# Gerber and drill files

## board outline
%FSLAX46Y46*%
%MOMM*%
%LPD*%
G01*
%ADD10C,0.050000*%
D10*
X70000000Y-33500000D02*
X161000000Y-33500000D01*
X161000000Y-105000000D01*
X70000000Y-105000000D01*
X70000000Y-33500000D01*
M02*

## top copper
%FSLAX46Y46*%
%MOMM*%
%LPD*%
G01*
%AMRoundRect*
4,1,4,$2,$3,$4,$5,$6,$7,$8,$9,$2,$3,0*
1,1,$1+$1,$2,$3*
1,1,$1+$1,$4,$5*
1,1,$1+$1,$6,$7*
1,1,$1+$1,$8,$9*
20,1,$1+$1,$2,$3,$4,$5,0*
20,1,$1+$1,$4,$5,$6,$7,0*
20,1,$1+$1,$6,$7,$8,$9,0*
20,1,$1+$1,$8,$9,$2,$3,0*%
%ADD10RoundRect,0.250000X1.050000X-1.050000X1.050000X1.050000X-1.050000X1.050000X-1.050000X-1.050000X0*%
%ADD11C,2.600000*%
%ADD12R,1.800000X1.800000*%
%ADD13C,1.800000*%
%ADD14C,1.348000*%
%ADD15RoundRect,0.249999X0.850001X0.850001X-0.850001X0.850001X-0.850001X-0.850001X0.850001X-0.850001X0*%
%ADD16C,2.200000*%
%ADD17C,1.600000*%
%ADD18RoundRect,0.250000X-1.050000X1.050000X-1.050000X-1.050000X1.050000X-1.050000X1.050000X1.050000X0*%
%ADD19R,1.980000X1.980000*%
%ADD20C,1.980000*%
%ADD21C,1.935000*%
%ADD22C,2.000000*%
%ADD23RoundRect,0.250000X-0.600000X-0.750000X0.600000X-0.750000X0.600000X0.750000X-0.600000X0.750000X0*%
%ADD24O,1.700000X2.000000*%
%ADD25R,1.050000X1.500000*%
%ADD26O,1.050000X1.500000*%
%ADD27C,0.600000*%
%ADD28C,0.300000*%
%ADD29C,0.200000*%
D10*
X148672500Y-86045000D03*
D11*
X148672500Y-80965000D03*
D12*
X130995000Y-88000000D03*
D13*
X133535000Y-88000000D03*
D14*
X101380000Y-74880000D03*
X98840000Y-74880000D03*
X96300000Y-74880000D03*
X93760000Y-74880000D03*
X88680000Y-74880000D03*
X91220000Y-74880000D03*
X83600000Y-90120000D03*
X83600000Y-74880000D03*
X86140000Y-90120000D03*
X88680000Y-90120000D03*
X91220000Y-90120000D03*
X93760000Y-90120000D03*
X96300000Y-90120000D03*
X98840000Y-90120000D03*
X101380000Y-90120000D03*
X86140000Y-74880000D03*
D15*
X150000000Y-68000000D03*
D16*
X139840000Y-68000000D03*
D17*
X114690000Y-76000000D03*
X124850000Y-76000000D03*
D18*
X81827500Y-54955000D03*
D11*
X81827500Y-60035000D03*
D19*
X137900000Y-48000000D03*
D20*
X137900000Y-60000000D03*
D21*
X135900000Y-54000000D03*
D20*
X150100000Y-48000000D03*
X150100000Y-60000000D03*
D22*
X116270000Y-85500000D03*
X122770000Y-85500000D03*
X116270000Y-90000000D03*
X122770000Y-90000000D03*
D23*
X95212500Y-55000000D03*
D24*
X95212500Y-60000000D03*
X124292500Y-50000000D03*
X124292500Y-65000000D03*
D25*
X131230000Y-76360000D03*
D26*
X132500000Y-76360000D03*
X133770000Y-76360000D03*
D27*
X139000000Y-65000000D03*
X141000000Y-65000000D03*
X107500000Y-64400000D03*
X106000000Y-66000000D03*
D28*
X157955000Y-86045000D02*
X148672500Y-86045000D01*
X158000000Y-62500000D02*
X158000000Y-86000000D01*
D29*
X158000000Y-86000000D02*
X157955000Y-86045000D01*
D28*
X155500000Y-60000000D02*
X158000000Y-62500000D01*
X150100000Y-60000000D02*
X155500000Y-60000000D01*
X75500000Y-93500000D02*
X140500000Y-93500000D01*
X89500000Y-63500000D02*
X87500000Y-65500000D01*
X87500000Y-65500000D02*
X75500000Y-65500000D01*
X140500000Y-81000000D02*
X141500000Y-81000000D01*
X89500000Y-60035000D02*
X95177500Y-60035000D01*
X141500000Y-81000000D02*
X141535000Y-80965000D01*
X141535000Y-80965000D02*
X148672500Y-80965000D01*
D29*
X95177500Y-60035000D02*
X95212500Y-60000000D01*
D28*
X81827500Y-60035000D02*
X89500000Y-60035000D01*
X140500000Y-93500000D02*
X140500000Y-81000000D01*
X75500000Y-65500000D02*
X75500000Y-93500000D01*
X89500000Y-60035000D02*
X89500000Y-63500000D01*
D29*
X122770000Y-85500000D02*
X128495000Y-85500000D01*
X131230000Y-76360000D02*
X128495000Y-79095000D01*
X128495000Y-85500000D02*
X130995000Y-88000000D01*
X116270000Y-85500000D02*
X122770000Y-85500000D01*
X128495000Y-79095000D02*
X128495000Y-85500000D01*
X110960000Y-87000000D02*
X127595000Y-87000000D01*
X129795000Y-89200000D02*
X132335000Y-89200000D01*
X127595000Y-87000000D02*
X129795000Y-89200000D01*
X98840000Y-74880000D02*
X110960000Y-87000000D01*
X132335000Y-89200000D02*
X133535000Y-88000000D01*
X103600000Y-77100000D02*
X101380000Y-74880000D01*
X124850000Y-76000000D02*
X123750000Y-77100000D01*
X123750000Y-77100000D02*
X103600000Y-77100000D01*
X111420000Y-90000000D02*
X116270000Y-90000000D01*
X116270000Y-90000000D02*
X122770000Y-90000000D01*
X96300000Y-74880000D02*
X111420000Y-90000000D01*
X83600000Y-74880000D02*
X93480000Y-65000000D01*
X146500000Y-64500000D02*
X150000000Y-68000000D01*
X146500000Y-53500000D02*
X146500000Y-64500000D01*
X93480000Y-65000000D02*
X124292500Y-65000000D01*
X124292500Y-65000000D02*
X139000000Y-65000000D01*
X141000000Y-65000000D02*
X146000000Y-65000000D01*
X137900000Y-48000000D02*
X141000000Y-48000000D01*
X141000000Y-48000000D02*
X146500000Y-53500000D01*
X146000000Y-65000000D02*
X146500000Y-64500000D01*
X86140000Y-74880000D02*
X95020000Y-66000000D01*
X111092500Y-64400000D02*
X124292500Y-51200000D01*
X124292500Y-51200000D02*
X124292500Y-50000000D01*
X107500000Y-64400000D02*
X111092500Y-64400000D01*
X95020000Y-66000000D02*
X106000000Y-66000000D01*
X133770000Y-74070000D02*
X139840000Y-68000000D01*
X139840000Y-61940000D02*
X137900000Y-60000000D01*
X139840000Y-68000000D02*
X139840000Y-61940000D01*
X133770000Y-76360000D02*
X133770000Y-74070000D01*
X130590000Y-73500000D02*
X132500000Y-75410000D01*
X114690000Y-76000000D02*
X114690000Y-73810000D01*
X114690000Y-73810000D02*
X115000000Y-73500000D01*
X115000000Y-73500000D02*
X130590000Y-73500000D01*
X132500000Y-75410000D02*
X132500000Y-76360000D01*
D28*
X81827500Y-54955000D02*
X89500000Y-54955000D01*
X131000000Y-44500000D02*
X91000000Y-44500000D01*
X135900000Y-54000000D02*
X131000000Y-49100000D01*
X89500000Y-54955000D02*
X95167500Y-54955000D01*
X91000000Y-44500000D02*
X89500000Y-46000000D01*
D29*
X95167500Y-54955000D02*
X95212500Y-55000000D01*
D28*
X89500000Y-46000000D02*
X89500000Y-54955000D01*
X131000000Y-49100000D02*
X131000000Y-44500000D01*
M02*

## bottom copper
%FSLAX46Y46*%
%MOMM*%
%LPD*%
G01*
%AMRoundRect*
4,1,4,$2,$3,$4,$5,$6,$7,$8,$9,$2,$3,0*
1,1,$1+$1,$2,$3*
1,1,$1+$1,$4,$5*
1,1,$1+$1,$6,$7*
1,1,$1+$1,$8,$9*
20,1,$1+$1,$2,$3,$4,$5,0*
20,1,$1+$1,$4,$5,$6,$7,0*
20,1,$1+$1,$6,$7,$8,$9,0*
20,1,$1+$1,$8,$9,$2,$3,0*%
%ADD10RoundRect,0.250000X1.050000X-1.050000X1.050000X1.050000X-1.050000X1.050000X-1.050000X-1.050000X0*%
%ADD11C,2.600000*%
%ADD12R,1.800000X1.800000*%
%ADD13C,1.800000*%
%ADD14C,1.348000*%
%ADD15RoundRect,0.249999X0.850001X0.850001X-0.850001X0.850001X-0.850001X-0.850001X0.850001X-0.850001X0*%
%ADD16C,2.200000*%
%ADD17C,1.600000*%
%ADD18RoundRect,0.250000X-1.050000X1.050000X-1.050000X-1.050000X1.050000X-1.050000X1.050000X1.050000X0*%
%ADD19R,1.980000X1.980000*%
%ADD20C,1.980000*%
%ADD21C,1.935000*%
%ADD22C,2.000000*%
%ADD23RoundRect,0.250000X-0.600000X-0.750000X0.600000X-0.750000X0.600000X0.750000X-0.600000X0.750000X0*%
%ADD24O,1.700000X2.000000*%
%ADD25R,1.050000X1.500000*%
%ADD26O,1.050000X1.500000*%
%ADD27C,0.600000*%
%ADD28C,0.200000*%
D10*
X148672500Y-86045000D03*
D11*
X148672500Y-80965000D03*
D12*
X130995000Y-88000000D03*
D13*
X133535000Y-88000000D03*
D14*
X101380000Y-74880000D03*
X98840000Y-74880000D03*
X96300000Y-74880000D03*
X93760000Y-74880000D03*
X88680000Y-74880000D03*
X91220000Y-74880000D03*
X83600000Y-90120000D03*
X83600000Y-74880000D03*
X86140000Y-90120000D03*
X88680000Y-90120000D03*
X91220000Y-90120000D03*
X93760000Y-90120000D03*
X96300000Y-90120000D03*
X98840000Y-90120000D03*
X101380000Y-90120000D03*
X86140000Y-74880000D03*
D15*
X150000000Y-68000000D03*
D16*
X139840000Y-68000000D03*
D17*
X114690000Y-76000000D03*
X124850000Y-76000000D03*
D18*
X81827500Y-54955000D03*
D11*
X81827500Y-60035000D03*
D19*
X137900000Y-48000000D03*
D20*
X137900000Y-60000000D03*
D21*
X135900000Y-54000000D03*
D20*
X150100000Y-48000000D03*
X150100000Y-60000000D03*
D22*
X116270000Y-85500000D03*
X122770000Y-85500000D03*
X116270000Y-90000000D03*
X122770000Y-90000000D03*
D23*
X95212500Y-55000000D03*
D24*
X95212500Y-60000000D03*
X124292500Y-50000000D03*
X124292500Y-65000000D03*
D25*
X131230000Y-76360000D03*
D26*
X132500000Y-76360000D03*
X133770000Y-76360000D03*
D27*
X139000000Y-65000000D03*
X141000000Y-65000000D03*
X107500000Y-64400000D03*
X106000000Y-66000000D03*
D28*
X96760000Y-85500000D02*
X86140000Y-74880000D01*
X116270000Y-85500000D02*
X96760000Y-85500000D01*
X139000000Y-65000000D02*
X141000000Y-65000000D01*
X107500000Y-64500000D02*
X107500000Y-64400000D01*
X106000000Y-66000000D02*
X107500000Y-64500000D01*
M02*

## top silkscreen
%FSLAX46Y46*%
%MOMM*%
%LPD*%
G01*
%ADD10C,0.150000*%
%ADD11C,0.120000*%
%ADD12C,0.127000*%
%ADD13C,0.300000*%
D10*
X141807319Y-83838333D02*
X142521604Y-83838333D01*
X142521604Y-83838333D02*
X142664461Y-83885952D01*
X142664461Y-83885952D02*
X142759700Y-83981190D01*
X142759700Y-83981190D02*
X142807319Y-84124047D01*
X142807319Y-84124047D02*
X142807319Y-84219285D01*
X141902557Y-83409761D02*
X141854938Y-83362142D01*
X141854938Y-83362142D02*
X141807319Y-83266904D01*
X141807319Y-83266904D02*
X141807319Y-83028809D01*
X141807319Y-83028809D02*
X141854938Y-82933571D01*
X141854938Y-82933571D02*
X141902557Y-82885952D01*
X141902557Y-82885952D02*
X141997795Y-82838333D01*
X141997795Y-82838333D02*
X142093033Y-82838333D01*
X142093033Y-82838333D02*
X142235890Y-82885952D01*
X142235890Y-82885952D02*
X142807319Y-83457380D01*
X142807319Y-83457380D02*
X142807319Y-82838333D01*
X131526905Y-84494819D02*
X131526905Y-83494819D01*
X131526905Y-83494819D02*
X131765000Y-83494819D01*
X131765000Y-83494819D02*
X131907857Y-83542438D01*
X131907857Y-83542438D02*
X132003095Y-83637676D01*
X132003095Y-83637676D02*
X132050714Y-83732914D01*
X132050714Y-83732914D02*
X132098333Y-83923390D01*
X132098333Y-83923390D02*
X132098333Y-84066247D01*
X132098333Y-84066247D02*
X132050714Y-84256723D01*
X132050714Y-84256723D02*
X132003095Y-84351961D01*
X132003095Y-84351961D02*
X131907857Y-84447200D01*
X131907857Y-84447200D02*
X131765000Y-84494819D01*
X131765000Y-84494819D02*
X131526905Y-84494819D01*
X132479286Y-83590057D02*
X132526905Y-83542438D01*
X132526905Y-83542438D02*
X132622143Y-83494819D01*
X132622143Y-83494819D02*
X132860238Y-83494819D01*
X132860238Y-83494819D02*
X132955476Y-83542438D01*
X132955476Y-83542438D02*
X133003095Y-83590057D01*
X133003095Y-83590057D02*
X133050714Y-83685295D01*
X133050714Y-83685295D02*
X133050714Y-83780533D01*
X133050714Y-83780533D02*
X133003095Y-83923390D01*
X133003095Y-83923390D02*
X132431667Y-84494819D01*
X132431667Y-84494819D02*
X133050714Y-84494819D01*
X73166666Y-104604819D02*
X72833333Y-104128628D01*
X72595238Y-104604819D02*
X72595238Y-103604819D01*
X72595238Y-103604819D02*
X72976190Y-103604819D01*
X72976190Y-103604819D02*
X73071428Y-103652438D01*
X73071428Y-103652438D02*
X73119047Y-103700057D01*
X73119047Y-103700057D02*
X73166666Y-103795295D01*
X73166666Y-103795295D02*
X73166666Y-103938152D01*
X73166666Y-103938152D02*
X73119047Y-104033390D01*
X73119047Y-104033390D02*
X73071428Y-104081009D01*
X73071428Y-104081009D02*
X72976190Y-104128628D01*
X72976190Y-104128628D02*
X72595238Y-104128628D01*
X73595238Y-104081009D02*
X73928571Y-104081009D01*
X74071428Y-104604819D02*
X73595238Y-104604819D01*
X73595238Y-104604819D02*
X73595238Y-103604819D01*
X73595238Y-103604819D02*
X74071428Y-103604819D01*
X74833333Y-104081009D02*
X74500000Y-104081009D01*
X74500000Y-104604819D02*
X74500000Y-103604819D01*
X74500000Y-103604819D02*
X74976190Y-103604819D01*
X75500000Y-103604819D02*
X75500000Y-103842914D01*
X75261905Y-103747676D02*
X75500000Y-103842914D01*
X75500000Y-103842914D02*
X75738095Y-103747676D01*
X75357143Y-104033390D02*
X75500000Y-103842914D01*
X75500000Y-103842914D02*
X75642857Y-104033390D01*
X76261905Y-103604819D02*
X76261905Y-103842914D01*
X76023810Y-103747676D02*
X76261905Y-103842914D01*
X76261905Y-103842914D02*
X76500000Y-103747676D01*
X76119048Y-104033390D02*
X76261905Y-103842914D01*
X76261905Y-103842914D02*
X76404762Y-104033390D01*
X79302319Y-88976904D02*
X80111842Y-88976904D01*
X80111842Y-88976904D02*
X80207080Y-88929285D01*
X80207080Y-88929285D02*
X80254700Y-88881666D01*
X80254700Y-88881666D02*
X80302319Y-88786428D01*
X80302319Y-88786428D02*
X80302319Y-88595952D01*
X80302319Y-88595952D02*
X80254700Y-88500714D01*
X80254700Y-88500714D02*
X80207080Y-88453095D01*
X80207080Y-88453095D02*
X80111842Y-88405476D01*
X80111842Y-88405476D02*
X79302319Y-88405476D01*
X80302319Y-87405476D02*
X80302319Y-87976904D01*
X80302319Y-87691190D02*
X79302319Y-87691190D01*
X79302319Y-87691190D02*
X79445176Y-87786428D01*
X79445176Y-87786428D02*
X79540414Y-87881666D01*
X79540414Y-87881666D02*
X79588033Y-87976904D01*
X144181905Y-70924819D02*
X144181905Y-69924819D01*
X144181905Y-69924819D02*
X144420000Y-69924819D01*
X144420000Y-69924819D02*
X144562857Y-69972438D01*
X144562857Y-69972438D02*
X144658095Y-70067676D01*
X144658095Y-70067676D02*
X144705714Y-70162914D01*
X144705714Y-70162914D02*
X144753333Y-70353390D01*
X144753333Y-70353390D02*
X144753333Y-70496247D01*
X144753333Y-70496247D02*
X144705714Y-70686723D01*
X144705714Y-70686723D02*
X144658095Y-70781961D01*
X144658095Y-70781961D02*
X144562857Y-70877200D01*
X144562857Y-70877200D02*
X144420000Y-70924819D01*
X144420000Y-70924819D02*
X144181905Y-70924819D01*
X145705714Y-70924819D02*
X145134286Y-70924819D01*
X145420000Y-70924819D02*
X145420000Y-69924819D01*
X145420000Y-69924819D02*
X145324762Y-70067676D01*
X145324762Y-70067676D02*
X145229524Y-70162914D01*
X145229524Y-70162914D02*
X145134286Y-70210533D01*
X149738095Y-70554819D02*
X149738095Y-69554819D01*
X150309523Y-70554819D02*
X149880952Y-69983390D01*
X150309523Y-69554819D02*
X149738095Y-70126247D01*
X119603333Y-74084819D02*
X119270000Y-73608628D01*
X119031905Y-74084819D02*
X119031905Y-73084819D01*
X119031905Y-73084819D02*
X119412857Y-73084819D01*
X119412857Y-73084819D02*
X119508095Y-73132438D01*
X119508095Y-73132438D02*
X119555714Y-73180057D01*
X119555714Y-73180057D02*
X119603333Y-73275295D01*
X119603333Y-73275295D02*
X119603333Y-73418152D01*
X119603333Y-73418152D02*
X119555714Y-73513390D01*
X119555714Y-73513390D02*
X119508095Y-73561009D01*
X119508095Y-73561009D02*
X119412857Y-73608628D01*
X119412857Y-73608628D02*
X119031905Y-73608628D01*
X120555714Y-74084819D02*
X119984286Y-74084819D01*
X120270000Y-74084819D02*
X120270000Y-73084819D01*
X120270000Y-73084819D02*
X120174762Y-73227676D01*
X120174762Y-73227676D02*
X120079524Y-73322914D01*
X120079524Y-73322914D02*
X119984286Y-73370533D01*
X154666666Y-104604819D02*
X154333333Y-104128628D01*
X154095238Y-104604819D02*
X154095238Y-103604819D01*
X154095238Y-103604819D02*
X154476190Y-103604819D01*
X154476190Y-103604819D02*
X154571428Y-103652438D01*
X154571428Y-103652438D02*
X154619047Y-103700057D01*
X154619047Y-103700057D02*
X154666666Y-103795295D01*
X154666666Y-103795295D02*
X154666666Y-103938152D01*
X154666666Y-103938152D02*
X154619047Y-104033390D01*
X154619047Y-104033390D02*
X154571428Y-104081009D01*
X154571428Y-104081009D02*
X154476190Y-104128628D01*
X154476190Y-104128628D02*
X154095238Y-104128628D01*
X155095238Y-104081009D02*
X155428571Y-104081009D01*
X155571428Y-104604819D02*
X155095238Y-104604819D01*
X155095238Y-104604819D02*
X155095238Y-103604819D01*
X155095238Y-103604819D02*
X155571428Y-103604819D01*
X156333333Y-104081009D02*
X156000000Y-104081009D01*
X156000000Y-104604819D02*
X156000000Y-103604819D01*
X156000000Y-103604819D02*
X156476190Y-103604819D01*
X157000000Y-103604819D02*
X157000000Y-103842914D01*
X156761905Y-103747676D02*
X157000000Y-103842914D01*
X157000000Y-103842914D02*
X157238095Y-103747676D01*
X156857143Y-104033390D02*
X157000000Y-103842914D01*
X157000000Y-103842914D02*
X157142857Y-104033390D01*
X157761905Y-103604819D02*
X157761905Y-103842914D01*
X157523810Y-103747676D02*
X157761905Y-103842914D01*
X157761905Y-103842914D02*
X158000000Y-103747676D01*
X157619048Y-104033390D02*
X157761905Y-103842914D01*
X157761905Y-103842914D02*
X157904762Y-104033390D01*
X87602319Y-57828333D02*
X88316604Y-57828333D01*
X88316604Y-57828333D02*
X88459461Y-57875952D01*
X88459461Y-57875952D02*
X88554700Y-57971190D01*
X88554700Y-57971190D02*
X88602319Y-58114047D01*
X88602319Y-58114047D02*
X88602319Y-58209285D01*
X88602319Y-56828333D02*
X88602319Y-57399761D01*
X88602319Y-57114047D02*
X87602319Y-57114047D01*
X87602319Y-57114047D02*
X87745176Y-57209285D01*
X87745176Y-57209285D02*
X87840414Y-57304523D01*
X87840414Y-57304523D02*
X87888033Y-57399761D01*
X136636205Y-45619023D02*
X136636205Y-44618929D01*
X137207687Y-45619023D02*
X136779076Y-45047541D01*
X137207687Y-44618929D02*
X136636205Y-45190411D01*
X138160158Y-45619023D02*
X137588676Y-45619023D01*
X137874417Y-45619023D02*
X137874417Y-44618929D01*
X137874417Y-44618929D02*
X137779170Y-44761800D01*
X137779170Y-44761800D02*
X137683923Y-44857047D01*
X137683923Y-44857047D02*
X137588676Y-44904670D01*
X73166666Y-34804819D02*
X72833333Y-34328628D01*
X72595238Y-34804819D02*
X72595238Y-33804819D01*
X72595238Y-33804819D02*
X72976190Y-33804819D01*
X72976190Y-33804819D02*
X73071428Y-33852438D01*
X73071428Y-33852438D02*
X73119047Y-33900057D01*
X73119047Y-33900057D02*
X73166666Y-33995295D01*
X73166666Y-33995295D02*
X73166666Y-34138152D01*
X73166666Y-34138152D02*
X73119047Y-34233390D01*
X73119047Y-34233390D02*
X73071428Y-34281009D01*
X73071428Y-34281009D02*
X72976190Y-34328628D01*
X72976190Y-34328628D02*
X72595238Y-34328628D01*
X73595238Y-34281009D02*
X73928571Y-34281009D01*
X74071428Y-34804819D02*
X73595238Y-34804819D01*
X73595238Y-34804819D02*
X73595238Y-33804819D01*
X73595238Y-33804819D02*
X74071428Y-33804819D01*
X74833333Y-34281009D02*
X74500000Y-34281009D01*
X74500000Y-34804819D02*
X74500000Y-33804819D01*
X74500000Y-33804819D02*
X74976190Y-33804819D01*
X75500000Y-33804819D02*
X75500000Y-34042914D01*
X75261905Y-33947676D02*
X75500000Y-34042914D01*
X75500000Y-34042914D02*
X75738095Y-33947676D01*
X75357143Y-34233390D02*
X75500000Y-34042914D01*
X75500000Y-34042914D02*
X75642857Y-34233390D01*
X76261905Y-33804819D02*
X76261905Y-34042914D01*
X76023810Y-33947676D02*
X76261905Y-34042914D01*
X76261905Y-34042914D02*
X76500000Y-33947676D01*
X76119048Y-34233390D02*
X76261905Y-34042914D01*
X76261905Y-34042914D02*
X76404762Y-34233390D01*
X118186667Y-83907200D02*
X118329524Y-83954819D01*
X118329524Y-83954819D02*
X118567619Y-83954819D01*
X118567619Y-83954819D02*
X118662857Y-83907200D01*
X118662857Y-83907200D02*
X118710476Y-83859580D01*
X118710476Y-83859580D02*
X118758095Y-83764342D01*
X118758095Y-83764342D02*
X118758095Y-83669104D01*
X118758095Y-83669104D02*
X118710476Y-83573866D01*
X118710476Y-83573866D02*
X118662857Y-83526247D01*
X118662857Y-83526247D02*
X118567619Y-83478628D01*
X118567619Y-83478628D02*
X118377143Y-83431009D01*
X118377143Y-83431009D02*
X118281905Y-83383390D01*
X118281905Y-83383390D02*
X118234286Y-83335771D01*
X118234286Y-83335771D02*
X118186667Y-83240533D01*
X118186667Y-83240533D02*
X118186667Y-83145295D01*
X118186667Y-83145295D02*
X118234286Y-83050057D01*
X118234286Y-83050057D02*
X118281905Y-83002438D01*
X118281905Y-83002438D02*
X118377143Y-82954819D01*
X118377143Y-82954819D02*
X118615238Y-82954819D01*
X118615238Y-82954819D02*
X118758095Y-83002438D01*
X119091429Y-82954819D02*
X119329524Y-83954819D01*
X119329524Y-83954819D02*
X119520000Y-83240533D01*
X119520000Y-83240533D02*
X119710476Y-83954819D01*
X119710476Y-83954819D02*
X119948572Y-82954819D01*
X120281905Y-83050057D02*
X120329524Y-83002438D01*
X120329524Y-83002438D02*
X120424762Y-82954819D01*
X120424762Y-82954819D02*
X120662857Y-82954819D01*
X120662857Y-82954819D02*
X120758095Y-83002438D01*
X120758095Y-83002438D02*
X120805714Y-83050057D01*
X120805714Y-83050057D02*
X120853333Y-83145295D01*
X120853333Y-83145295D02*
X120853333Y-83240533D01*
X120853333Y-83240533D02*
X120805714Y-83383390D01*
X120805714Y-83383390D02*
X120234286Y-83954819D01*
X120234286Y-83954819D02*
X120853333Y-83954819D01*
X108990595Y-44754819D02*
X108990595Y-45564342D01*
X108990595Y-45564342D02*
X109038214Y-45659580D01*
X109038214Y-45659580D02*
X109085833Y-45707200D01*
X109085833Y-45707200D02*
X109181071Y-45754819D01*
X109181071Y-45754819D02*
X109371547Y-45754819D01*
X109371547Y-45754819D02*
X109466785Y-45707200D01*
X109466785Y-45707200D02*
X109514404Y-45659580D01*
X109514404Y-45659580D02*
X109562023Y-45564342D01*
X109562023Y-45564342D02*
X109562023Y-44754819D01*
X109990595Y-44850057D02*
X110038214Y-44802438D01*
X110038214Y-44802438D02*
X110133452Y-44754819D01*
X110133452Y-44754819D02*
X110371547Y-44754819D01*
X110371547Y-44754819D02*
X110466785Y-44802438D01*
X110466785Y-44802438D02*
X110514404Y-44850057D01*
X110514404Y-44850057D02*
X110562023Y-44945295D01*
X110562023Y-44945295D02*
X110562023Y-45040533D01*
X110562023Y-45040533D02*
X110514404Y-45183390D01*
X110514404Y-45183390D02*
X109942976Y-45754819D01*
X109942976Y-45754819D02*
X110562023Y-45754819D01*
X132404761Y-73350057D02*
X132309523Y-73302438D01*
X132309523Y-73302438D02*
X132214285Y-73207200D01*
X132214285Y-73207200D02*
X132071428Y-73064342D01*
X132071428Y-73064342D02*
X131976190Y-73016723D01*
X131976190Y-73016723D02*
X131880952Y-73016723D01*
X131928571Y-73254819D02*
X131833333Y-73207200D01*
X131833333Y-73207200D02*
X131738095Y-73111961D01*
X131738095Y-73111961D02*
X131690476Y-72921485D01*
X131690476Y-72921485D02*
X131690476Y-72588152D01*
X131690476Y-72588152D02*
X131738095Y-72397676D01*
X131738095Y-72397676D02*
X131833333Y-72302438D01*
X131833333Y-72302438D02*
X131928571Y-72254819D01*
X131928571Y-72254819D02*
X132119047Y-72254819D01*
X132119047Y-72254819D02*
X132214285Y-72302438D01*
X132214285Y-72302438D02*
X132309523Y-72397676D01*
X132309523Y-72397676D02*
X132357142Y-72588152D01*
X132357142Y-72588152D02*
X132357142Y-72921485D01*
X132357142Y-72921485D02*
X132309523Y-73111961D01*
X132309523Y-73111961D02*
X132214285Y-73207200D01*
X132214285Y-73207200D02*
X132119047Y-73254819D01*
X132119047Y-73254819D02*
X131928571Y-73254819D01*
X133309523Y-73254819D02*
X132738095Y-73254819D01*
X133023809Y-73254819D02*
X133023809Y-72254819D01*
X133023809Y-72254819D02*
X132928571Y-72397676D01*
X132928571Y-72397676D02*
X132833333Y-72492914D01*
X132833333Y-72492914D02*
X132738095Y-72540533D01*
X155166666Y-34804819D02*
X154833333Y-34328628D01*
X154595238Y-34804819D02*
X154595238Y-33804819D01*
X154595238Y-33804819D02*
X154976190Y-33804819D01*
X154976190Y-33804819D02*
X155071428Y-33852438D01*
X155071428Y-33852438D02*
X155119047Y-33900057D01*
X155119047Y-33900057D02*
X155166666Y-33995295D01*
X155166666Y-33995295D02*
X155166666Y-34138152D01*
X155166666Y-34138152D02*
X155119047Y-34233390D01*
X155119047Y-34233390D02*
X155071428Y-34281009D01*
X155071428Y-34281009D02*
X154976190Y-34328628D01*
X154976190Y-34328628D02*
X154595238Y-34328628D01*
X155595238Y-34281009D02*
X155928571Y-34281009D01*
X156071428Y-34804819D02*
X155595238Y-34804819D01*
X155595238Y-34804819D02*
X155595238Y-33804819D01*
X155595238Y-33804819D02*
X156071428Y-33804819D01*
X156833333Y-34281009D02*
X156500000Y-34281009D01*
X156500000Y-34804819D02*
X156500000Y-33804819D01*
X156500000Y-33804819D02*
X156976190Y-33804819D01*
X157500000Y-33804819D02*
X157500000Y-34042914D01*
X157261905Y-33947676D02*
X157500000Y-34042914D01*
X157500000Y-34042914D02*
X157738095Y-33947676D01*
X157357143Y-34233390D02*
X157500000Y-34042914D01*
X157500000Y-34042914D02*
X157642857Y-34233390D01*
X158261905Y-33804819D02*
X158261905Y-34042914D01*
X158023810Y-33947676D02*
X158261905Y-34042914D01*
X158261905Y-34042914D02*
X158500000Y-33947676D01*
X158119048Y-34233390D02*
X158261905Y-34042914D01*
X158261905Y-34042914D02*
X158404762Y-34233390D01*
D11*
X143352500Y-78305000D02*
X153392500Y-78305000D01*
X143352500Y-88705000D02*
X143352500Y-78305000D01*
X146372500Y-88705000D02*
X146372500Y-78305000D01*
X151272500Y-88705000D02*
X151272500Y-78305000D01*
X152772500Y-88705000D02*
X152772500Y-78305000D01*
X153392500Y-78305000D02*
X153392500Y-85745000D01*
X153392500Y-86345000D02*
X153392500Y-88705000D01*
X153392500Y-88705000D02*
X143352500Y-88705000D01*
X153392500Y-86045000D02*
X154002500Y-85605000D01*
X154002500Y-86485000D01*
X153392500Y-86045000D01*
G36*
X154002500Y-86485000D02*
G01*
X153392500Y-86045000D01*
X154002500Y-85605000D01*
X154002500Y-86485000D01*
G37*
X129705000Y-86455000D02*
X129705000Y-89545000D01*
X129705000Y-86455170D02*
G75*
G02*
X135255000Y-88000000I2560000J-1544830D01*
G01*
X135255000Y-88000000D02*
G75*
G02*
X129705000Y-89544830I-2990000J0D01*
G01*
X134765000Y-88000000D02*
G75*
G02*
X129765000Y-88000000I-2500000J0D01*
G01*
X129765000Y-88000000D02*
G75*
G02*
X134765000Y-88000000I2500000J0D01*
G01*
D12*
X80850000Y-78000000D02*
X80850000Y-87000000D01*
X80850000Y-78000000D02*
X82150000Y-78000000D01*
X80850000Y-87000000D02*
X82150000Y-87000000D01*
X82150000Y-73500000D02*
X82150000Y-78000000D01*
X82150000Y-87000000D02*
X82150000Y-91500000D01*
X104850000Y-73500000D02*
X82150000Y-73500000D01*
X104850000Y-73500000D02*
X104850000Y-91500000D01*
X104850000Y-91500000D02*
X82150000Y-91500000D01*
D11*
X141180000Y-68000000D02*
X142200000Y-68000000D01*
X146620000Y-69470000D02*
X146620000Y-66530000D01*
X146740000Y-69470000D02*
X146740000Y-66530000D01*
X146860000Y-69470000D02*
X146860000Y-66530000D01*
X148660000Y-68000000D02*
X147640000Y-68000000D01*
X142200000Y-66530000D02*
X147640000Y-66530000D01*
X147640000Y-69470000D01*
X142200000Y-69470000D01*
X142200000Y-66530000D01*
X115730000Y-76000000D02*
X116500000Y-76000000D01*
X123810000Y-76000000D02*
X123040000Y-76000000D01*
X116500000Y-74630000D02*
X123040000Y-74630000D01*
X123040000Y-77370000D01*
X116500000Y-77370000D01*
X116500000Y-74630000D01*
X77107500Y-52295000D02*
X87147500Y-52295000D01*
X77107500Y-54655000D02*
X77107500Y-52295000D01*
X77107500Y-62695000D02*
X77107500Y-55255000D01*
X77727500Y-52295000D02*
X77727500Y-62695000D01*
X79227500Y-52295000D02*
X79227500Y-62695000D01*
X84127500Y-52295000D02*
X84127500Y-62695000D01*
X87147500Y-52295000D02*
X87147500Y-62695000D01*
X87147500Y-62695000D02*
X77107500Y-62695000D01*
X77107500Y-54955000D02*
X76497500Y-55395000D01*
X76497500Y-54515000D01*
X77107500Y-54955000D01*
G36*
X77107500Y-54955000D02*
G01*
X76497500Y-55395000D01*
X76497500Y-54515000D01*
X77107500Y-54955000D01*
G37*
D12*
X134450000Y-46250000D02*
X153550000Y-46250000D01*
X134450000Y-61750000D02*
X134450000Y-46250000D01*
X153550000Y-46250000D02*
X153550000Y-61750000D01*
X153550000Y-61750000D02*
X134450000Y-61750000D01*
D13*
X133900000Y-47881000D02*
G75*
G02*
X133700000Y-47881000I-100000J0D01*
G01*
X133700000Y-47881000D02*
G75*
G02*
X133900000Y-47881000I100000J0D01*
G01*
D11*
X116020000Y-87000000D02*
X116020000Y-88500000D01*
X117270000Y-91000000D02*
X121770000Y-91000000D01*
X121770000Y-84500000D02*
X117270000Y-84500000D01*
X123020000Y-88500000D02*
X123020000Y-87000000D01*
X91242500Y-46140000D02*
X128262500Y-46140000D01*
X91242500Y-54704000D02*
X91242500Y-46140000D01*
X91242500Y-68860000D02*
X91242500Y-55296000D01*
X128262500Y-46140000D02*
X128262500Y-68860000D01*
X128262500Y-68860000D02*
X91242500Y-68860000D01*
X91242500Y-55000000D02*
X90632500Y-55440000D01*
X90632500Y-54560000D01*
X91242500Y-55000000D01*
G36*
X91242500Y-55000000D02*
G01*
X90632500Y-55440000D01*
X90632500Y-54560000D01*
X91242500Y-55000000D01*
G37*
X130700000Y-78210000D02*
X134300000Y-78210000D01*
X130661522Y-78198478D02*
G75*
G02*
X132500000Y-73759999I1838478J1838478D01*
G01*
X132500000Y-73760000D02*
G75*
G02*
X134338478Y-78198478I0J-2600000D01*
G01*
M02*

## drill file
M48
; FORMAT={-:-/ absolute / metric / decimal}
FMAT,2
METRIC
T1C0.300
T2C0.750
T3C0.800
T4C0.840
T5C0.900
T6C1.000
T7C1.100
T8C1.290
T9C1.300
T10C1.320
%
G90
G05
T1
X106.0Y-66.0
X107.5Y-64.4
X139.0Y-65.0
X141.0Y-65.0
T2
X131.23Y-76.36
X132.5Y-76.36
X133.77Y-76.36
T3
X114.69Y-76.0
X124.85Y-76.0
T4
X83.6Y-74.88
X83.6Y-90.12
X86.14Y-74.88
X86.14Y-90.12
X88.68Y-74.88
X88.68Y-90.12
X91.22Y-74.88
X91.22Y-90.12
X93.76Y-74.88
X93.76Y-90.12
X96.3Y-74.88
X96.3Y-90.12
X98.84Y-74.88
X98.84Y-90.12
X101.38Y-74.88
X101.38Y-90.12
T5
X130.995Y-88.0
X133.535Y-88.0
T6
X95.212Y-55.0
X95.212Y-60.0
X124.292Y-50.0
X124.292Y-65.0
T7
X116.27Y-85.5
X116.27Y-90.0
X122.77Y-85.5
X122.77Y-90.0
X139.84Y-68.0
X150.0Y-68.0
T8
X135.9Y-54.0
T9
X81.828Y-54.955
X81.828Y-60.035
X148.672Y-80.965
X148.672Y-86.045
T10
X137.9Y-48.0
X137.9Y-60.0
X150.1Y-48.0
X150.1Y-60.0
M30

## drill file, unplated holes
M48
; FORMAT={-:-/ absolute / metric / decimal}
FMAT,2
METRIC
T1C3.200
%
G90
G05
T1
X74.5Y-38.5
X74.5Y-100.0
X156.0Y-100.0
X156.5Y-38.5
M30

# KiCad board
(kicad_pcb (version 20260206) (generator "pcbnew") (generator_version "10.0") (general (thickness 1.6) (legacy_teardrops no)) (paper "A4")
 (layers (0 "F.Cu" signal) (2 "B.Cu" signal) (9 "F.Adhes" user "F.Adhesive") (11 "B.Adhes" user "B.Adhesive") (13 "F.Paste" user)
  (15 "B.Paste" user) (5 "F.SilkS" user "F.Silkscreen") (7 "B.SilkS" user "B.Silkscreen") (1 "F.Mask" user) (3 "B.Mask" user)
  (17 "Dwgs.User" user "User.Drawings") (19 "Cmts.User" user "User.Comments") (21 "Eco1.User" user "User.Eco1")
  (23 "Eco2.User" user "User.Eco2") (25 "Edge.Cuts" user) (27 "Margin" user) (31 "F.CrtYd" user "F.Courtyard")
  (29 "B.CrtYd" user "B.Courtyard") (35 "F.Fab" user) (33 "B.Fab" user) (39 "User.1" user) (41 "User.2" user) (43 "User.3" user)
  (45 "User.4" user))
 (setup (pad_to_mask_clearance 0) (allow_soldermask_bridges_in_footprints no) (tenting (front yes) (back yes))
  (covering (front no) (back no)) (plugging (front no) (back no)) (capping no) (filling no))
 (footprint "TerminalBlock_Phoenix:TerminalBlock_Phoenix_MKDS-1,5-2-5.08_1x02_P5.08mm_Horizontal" (layer "F.Cu") (at 148.6725 86.045 90)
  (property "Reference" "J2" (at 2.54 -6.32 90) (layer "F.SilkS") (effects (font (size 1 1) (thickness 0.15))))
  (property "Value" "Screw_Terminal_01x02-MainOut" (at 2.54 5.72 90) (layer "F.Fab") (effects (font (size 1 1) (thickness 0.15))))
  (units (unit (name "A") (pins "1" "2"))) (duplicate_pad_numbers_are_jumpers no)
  (fp_line (start 7.74 -5.32) (end 7.74 4.72) (stroke (width 0.12) (type solid)) (layer "F.SilkS"))
  (fp_line (start -2.66 -5.32) (end 7.74 -5.32) (stroke (width 0.12) (type solid)) (layer "F.SilkS"))
  (fp_line (start -2.66 -2.3) (end 7.74 -2.3) (stroke (width 0.12) (type solid)) (layer "F.SilkS"))
  (fp_line (start -2.66 2.6) (end 7.74 2.6) (stroke (width 0.12) (type solid)) (layer "F.SilkS"))
  (fp_line (start -2.66 4.1) (end 7.74 4.1) (stroke (width 0.12) (type solid)) (layer "F.SilkS"))
  (fp_line (start 7.74 4.72) (end 0.3 4.72) (stroke (width 0.12) (type solid)) (layer "F.SilkS"))
  (fp_line (start -0.3 4.72) (end -2.66 4.72) (stroke (width 0.12) (type solid)) (layer "F.SilkS"))
  (fp_line (start -2.66 4.72) (end -2.66 -5.32) (stroke (width 0.12) (type solid)) (layer "F.SilkS"))
  (fp_poly (pts (xy 0 4.72) (xy 0.44 5.33) (xy -0.44 5.33)) (stroke (width 0.12) (type solid)) (fill yes) (layer "F.SilkS"))
  (pad "1" thru_hole roundrect (at 0 0 90) (size 2.6 2.6) (drill 1.3) (layers "*.Cu" "*.Mask") (remove_unused_layers no)
   (roundrect_rratio 0.096154) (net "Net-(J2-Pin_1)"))
  (pad "2" thru_hole circle (at 5.08 0 90) (size 2.6 2.6) (drill 1.3) (layers "*.Cu" "*.Mask") (remove_unused_layers no)
   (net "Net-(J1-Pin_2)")))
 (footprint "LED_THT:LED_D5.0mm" (layer "F.Cu") (at 130.995 88)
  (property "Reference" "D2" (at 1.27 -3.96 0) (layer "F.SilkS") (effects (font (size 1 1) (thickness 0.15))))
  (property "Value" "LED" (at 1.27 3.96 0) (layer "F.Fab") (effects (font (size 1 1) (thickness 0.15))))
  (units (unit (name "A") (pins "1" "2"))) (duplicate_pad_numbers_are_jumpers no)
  (fp_line (start -1.29 -1.545) (end -1.29 1.545) (stroke (width 0.12) (type solid)) (layer "F.SilkS"))
  (fp_arc (start -1.29 -1.54483) (mid 2.071779 -2.880495) (end 4.26 0) (stroke (width 0.12) (type solid)) (layer "F.SilkS"))
  (fp_arc (start 4.26 0) (mid 2.071779 2.880495) (end -1.29 1.54483) (stroke (width 0.12) (type solid)) (layer "F.SilkS"))
  (fp_circle (center 1.27 0) (end 3.77 0) (stroke (width 0.12) (type solid)) (fill no) (layer "F.SilkS"))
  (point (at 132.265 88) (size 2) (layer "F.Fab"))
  (pad "1" thru_hole rect (at 0 0) (size 1.8 1.8) (drill 0.9) (layers "*.Cu" "*.Mask") (remove_unused_layers no) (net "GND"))
  (pad "2" thru_hole circle (at 2.54 0) (size 1.8 1.8) (drill 0.9) (layers "*.Cu" "*.Mask") (remove_unused_layers no) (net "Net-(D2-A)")))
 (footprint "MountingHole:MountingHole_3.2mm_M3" (layer "F.Cu") (at 74.5 100 180)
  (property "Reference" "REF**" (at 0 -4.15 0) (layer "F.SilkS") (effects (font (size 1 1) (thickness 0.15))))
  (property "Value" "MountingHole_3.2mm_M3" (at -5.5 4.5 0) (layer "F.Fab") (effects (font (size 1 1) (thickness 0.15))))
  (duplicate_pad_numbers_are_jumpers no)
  (pad "" np_thru_hole circle (at 0 0 180) (size 3.2 3.2) (drill 3.2) (layers "*.Cu" "*.Mask")))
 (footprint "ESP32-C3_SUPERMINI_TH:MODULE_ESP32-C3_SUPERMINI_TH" (layer "F.Cu") (at 93.5 82.5 90)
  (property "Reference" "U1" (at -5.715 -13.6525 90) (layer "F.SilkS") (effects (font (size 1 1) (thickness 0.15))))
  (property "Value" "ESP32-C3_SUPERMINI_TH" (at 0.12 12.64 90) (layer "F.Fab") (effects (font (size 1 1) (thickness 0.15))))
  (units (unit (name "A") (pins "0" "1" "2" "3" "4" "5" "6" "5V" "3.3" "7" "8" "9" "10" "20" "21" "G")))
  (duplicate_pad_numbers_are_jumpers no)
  (fp_line (start 4.5 -12.65) (end -4.5 -12.65) (stroke (width 0.127) (type solid)) (layer "F.SilkS"))
  (fp_line (start 4.5 -12.65) (end 4.5 -11.35) (stroke (width 0.127) (type solid)) (layer "F.SilkS"))
  (fp_line (start -4.5 -12.65) (end -4.5 -11.35) (stroke (width 0.127) (type solid)) (layer "F.SilkS"))
  (fp_line (start 9 -11.35) (end 4.5 -11.35) (stroke (width 0.127) (type solid)) (layer "F.SilkS"))
  (fp_line (start -4.5 -11.35) (end -9 -11.35) (stroke (width 0.127) (type solid)) (layer "F.SilkS"))
  (fp_line (start 9 11.35) (end 9 -11.35) (stroke (width 0.127) (type solid)) (layer "F.SilkS"))
  (fp_line (start 9 11.35) (end -9 11.35) (stroke (width 0.127) (type solid)) (layer "F.SilkS"))
  (fp_line (start -9 11.35) (end -9 -11.35) (stroke (width 0.127) (type solid)) (layer "F.SilkS"))
  (pad "0" thru_hole circle (at 7.62 7.88 90) (size 1.348 1.348) (drill 0.84) (layers "*.Cu" "*.Mask") (remove_unused_layers no)
   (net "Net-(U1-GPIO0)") (solder_mask_margin 0.102))
  (pad "1" thru_hole circle (at 7.62 5.34 90) (size 1.348 1.348) (drill 0.84) (layers "*.Cu" "*.Mask") (remove_unused_layers no)
   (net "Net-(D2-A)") (solder_mask_margin 0.102))
  (pad "2" thru_hole circle (at 7.62 2.8 90) (size 1.348 1.348) (drill 0.84) (layers "*.Cu" "*.Mask") (remove_unused_layers no)
   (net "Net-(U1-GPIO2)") (solder_mask_margin 0.102))
  (pad "3" thru_hole circle (at 7.62 0.26 90) (size 1.348 1.348) (drill 0.84) (layers "*.Cu" "*.Mask") (remove_unused_layers no)
   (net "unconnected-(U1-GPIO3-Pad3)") (solder_mask_margin 0.102))
  (pad "3.3" thru_hole circle (at 7.62 -4.82 90) (size 1.348 1.348) (drill 0.84) (layers "*.Cu" "*.Mask") (remove_unused_layers no)
   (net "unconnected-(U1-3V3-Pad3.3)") (solder_mask_margin 0.102))
  (pad "4" thru_hole circle (at 7.62 -2.28 90) (size 1.348 1.348) (drill 0.84) (layers "*.Cu" "*.Mask") (remove_unused_layers no)
   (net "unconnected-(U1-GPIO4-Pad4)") (solder_mask_margin 0.102))
  (pad "5" thru_hole circle (at -7.62 -9.9 90) (size 1.348 1.348) (drill 0.84) (layers "*.Cu" "*.Mask") (remove_unused_layers no)
   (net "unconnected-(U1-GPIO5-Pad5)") (solder_mask_margin 0.102))
  (pad "5V" thru_hole circle (at 7.62 -9.9 90) (size 1.348 1.348) (drill 0.84) (layers "*.Cu" "*.Mask") (remove_unused_layers no)
   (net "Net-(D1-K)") (solder_mask_margin 0.102))
  (pad "6" thru_hole circle (at -7.62 -7.36 90) (size 1.348 1.348) (drill 0.84) (layers "*.Cu" "*.Mask") (remove_unused_layers no)
   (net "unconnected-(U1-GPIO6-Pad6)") (solder_mask_margin 0.102))
  (pad "7" thru_hole circle (at -7.62 -4.82 90) (size 1.348 1.348) (drill 0.84) (layers "*.Cu" "*.Mask") (remove_unused_layers no)
   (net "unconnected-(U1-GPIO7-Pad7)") (solder_mask_margin 0.102))
  (pad "8" thru_hole circle (at -7.62 -2.28 90) (size 1.348 1.348) (drill 0.84) (layers "*.Cu" "*.Mask") (remove_unused_layers no)
   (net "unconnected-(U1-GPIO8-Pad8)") (solder_mask_margin 0.102))
  (pad "9" thru_hole circle (at -7.62 0.26 90) (size 1.348 1.348) (drill 0.84) (layers "*.Cu" "*.Mask") (remove_unused_layers no)
   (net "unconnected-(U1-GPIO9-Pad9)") (solder_mask_margin 0.102))
  (pad "10" thru_hole circle (at -7.62 2.8 90) (size 1.348 1.348) (drill 0.84) (layers "*.Cu" "*.Mask") (remove_unused_layers no)
   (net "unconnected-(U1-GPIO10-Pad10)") (solder_mask_margin 0.102))
  (pad "20" thru_hole circle (at -7.62 5.34 90) (size 1.348 1.348) (drill 0.84) (layers "*.Cu" "*.Mask") (remove_unused_layers no)
   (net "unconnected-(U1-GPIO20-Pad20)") (solder_mask_margin 0.102))
  (pad "21" thru_hole circle (at -7.62 7.88 90) (size 1.348 1.348) (drill 0.84) (layers "*.Cu" "*.Mask") (remove_unused_layers no)
   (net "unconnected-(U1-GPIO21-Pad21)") (solder_mask_margin 0.102))
  (pad "G" thru_hole circle (at 7.62 -7.36 90) (size 1.348 1.348) (drill 0.84) (layers "*.Cu" "*.Mask") (remove_unused_layers no)
   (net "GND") (solder_mask_margin 0.102)))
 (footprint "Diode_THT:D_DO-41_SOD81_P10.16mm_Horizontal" (layer "F.Cu") (at 150 68 180)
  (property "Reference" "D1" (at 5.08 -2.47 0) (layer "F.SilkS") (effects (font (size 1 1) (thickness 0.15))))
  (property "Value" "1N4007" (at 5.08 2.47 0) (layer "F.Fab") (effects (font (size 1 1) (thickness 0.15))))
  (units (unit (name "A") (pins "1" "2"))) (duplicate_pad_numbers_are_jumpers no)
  (fp_line (start 8.82 0) (end 7.8 0) (stroke (width 0.12) (type solid)) (layer "F.SilkS"))
  (fp_line (start 3.38 -1.47) (end 3.38 1.47) (stroke (width 0.12) (type solid)) (layer "F.SilkS"))
  (fp_line (start 3.26 -1.47) (end 3.26 1.47) (stroke (width 0.12) (type solid)) (layer "F.SilkS"))
  (fp_line (start 3.14 -1.47) (end 3.14 1.47) (stroke (width 0.12) (type solid)) (layer "F.SilkS"))
  (fp_line (start 1.34 0) (end 2.36 0) (stroke (width 0.12) (type solid)) (layer "F.SilkS"))
  (fp_rect (start 2.36 -1.47) (end 7.8 1.47) (stroke (width 0.12) (type solid)) (fill no) (layer "F.SilkS"))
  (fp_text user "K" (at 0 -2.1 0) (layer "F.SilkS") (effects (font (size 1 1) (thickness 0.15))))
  (pad "1" thru_hole roundrect (at 0 0 180) (size 2.2 2.2) (drill 1.1) (layers "*.Cu" "*.Mask") (remove_unused_layers no)
   (roundrect_rratio 0.113636) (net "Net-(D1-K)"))
  (pad "2" thru_hole circle (at 10.16 0 180) (size 2.2 2.2) (drill 1.1) (layers "*.Cu" "*.Mask") (remove_unused_layers no)
   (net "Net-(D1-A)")))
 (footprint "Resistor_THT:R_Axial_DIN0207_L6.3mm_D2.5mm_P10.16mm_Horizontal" (layer "F.Cu") (at 114.69 76)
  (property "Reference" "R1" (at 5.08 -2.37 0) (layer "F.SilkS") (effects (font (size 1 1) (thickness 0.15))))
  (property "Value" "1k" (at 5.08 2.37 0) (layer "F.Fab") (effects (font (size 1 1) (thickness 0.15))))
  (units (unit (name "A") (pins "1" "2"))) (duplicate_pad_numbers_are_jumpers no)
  (fp_line (start 1.04 0) (end 1.81 0) (stroke (width 0.12) (type solid)) (layer "F.SilkS"))
  (fp_line (start 9.12 0) (end 8.35 0) (stroke (width 0.12) (type solid)) (layer "F.SilkS"))
  (fp_rect (start 1.81 -1.37) (end 8.35 1.37) (stroke (width 0.12) (type solid)) (fill no) (layer "F.SilkS"))
  (pad "1" thru_hole circle (at 0 0) (size 1.6 1.6) (drill 0.8) (layers "*.Cu" "*.Mask") (remove_unused_layers no) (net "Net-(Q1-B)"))
  (pad "2" thru_hole circle (at 10.16 0) (size 1.6 1.6) (drill 0.8) (layers "*.Cu" "*.Mask") (remove_unused_layers no)
   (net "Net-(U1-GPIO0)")))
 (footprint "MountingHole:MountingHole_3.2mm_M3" (layer "F.Cu") (at 156 100 180)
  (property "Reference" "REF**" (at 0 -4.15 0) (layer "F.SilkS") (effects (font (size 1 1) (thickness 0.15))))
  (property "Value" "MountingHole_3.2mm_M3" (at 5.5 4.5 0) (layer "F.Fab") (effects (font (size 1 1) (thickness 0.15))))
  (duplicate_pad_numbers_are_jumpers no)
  (pad "" np_thru_hole circle (at 0 0 180) (size 3.2 3.2) (drill 3.2) (layers "*.Cu" "*.Mask")))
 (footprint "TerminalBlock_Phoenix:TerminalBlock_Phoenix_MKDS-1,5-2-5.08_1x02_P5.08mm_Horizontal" (layer "F.Cu") (at 81.8275 54.955 -90)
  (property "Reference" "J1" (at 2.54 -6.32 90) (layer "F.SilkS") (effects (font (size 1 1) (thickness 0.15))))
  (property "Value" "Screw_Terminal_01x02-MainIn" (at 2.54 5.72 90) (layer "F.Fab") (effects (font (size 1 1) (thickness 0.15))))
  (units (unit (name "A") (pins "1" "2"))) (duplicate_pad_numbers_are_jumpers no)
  (fp_line (start -2.66 4.72) (end -2.66 -5.32) (stroke (width 0.12) (type solid)) (layer "F.SilkS"))
  (fp_line (start -0.3 4.72) (end -2.66 4.72) (stroke (width 0.12) (type solid)) (layer "F.SilkS"))
  (fp_line (start 7.74 4.72) (end 0.3 4.72) (stroke (width 0.12) (type solid)) (layer "F.SilkS"))
  (fp_line (start -2.66 4.1) (end 7.74 4.1) (stroke (width 0.12) (type solid)) (layer "F.SilkS"))
  (fp_line (start -2.66 2.6) (end 7.74 2.6) (stroke (width 0.12) (type solid)) (layer "F.SilkS"))
  (fp_line (start -2.66 -2.3) (end 7.74 -2.3) (stroke (width 0.12) (type solid)) (layer "F.SilkS"))
  (fp_line (start -2.66 -5.32) (end 7.74 -5.32) (stroke (width 0.12) (type solid)) (layer "F.SilkS"))
  (fp_line (start 7.74 -5.32) (end 7.74 4.72) (stroke (width 0.12) (type solid)) (layer "F.SilkS"))
  (fp_poly (pts (xy 0 4.72) (xy 0.44 5.33) (xy -0.44 5.33)) (stroke (width 0.12) (type solid)) (fill yes) (layer "F.SilkS"))
  (pad "1" thru_hole roundrect (at 0 0 270) (size 2.6 2.6) (drill 1.3) (layers "*.Cu" "*.Mask") (remove_unused_layers no)
   (roundrect_rratio 0.096154) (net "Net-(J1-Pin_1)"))
  (pad "2" thru_hole circle (at 5.08 0 270) (size 2.6 2.6) (drill 1.3) (layers "*.Cu" "*.Mask") (remove_unused_layers no)
   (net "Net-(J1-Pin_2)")))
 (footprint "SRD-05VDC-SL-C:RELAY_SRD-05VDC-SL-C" (layer "F.Cu") (at 144 54)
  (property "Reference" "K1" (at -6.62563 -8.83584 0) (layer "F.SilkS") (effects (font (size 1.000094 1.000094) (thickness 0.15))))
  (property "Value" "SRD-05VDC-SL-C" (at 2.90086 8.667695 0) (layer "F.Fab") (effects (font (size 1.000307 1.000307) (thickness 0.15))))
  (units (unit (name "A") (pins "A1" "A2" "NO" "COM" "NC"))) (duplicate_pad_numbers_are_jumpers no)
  (fp_line (start -9.55 -7.75) (end 9.55 -7.75) (stroke (width 0.127) (type solid)) (layer "F.SilkS"))
  (fp_line (start -9.55 7.75) (end -9.55 -7.75) (stroke (width 0.127) (type solid)) (layer "F.SilkS"))
  (fp_line (start 9.55 -7.75) (end 9.55 7.75) (stroke (width 0.127) (type solid)) (layer "F.SilkS"))
  (fp_line (start 9.55 7.75) (end -9.55 7.75) (stroke (width 0.127) (type solid)) (layer "F.SilkS"))
  (fp_circle (center -10.2 -6.119) (end -10.1 -6.119) (stroke (width 0.3) (type solid)) (fill no) (layer "F.SilkS"))
  (pad "A1" thru_hole rect (at -6.1 -6) (size 1.98 1.98) (drill 1.32) (layers "*.Cu" "*.Mask") (remove_unused_layers no) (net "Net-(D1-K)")
   (solder_mask_margin 0.102))
  (pad "A2" thru_hole circle (at -6.1 6) (size 1.98 1.98) (drill 1.32) (layers "*.Cu" "*.Mask") (remove_unused_layers no) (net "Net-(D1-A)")
   (solder_mask_margin 0.102))
  (pad "COM" thru_hole circle (at -8.1 0) (size 1.935 1.935) (drill 1.29) (layers "*.Cu" "*.Mask") (remove_unused_layers no)
   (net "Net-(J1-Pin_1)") (solder_mask_margin 0.102))
  (pad "NC" thru_hole circle (at 6.1 -6) (size 1.98 1.98) (drill 1.32) (layers "*.Cu" "*.Mask") (remove_unused_layers no)
   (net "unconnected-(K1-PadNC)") (solder_mask_margin 0.102))
  (pad "NO" thru_hole circle (at 6.1 6) (size 1.98 1.98) (drill 1.32) (layers "*.Cu" "*.Mask") (remove_unused_layers no)
   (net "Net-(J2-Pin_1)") (solder_mask_margin 0.102)))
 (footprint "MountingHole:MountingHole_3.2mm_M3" (layer "F.Cu") (at 74.5 38.5)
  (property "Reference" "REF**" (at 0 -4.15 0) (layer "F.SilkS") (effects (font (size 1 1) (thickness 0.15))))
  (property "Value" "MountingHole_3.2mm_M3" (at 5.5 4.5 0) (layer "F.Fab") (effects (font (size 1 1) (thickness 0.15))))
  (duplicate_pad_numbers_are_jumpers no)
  (pad "" np_thru_hole circle (at 0 0) (size 3.2 3.2) (drill 3.2) (layers "*.Cu" "*.Mask")))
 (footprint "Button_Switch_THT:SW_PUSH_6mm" (layer "F.Cu") (at 116.27 85.5)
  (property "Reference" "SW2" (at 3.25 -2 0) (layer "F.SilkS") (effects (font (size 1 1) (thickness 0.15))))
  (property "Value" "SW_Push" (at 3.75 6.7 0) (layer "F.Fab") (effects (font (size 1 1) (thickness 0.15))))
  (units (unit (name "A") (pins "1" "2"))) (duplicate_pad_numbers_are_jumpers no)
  (fp_line (start -0.25 1.5) (end -0.25 3) (stroke (width 0.12) (type solid)) (layer "F.SilkS"))
  (fp_line (start 1 5.5) (end 5.5 5.5) (stroke (width 0.12) (type solid)) (layer "F.SilkS"))
  (fp_line (start 5.5 -1) (end 1 -1) (stroke (width 0.12) (type solid)) (layer "F.SilkS"))
  (fp_line (start 6.75 3) (end 6.75 1.5) (stroke (width 0.12) (type solid)) (layer "F.SilkS"))
  (pad "1" thru_hole circle (at 0 0 90) (size 2 2) (drill 1.1) (layers "*.Cu" "*.Mask") (remove_unused_layers no) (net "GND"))
  (pad "1" thru_hole circle (at 6.5 0 90) (size 2 2) (drill 1.1) (layers "*.Cu" "*.Mask") (remove_unused_layers no) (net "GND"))
  (pad "2" thru_hole circle (at 0 4.5 90) (size 2 2) (drill 1.1) (layers "*.Cu" "*.Mask") (remove_unused_layers no) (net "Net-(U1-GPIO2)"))
  (pad "2" thru_hole circle (at 6.5 4.5 90) (size 2 2) (drill 1.1) (layers "*.Cu" "*.Mask") (remove_unused_layers no) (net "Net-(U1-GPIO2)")))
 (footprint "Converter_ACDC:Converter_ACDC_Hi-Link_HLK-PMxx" (layer "F.Cu") (at 95.2125 55)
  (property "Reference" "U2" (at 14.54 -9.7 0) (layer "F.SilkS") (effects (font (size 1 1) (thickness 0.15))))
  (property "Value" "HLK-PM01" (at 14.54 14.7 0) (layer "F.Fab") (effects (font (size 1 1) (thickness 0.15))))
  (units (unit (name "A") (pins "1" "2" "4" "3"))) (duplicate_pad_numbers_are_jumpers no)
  (fp_line (start -3.97 -8.86) (end 33.05 -8.86) (stroke (width 0.12) (type solid)) (layer "F.SilkS"))
  (fp_line (start -3.97 -0.296) (end -3.97 -8.86) (stroke (width 0.12) (type solid)) (layer "F.SilkS"))
  (fp_line (start -3.97 13.86) (end -3.97 0.296) (stroke (width 0.12) (type solid)) (layer "F.SilkS"))
  (fp_line (start 33.05 -8.86) (end 33.05 13.86) (stroke (width 0.12) (type solid)) (layer "F.SilkS"))
  (fp_line (start 33.05 13.86) (end -3.97 13.86) (stroke (width 0.12) (type solid)) (layer "F.SilkS"))
  (fp_poly (pts (xy -3.97 0) (xy -4.58 0.44) (xy -4.58 -0.44)) (stroke (width 0.12) (type solid)) (fill yes) (layer "F.SilkS"))
  (pad "1" thru_hole roundrect (at 0 0) (size 1.7 2) (drill 1) (layers "*.Cu" "*.Mask") (remove_unused_layers no)
   (roundrect_rratio 0.147059) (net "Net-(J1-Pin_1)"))
  (pad "2" thru_hole oval (at 0 5) (size 1.7 2) (drill 1) (layers "*.Cu" "*.Mask") (remove_unused_layers no) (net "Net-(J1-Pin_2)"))
  (pad "3" thru_hole oval (at 29.08 -5) (size 1.7 2) (drill 1) (layers "*.Cu" "*.Mask") (remove_unused_layers no) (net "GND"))
  (pad "4" thru_hole oval (at 29.08 10) (size 1.7 2) (drill 1) (layers "*.Cu" "*.Mask") (remove_unused_layers no) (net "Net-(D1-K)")))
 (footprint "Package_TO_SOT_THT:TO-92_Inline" (layer "F.Cu") (at 131.23 76.36)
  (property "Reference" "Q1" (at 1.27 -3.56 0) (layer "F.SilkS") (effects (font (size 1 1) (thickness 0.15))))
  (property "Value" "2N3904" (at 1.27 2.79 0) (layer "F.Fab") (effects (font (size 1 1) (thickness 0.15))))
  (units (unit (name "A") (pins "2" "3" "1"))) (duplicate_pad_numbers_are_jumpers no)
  (fp_line (start -0.53 1.85) (end 3.07 1.85) (stroke (width 0.12) (type solid)) (layer "F.SilkS"))
  (fp_arc (start -0.568478 1.838478) (mid -1.132087 -0.994977) (end 1.27 -2.6) (stroke (width 0.12) (type solid)) (layer "F.SilkS"))
  (fp_arc (start 1.27 -2.6) (mid 3.672087 -0.994977) (end 3.108478 1.838478) (stroke (width 0.12) (type solid)) (layer "F.SilkS"))
  (pad "1" thru_hole rect (at 0 0) (size 1.05 1.5) (drill 0.75) (layers "*.Cu" "*.Mask") (remove_unused_layers no) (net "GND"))
  (pad "2" thru_hole oval (at 1.27 0) (size 1.05 1.5) (drill 0.75) (layers "*.Cu" "*.Mask") (remove_unused_layers no) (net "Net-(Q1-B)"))
  (pad "3" thru_hole oval (at 2.54 0) (size 1.05 1.5) (drill 0.75) (layers "*.Cu" "*.Mask") (remove_unused_layers no) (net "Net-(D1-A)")))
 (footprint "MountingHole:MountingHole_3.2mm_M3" (layer "F.Cu") (at 156.5 38.5)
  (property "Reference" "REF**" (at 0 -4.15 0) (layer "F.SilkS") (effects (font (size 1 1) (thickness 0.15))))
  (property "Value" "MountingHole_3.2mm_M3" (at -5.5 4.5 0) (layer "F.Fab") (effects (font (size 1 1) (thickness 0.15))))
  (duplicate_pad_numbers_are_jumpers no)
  (pad "" np_thru_hole circle (at 0 0) (size 3.2 3.2) (drill 3.2) (layers "*.Cu" "*.Mask")))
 (gr_rect (start 70 33.5) (end 161 105) (stroke (width 0.05) (type default)) (fill no) (layer "Edge.Cuts"))
 (segment (start 157.955 86.045) (end 148.6725 86.045) (width 0.3) (layer "F.Cu") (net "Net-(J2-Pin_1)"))
 (segment (start 158 62.5) (end 158 86) (width 0.3) (layer "F.Cu") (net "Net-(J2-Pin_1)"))
 (segment (start 158 86) (end 157.955 86.045) (width 0.2) (layer "F.Cu") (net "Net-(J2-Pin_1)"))
 (segment (start 155.5 60) (end 158 62.5) (width 0.3) (layer "F.Cu") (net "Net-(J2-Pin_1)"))
 (segment (start 150.1 60) (end 155.5 60) (width 0.3) (layer "F.Cu") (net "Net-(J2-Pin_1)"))
 (segment (start 75.5 93.5) (end 140.5 93.5) (width 0.3) (layer "F.Cu") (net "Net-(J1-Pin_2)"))
 (segment (start 89.5 63.5) (end 87.5 65.5) (width 0.3) (layer "F.Cu") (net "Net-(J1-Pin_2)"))
 (segment (start 87.5 65.5) (end 75.5 65.5) (width 0.3) (layer "F.Cu") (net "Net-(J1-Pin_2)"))
 (segment (start 140.5 81) (end 141.5 81) (width 0.3) (layer "F.Cu") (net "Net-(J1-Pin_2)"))
 (segment (start 89.5 60.035) (end 95.1775 60.035) (width 0.3) (layer "F.Cu") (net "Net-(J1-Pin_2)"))
 (segment (start 141.5 81) (end 141.535 80.965) (width 0.3) (layer "F.Cu") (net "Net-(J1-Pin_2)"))
 (segment (start 141.535 80.965) (end 148.6725 80.965) (width 0.3) (layer "F.Cu") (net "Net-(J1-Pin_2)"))
 (segment (start 95.1775 60.035) (end 95.2125 60) (width 0.2) (layer "F.Cu") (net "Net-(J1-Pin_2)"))
 (segment (start 81.8275 60.035) (end 89.5 60.035) (width 0.3) (layer "F.Cu") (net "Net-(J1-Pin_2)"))
 (segment (start 140.5 93.5) (end 140.5 81) (width 0.3) (layer "F.Cu") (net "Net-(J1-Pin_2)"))
 (segment (start 75.5 65.5) (end 75.5 93.5) (width 0.3) (layer "F.Cu") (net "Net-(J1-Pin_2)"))
 (segment (start 89.5 60.035) (end 89.5 63.5) (width 0.3) (layer "F.Cu") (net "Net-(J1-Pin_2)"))
 (segment (start 122.77 85.5) (end 128.495 85.5) (width 0.2) (layer "F.Cu") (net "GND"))
 (segment (start 86.14 74.88) (end 95.02 66) (width 0.2) (layer "F.Cu") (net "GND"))
 (segment (start 111.0925 64.4) (end 124.2925 51.2) (width 0.2) (layer "F.Cu") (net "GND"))
 (segment (start 124.2925 51.2) (end 124.2925 50) (width 0.2) (layer "F.Cu") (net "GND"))
 (segment (start 131.23 76.36) (end 128.495 79.095) (width 0.2) (layer "F.Cu") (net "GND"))
 (segment (start 107.5 64.4) (end 111.0925 64.4) (width 0.2) (layer "F.Cu") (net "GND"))
 (segment (start 128.495 85.5) (end 130.995 88) (width 0.2) (layer "F.Cu") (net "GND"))
 (segment (start 116.27 85.5) (end 122.77 85.5) (width 0.2) (layer "F.Cu") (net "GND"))
 (segment (start 128.495 79.095) (end 128.495 85.5) (width 0.2) (layer "F.Cu") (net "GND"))
 (segment (start 95.02 66) (end 106 66) (width 0.2) (layer "F.Cu") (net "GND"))
 (via (at 107.5 64.4) (size 0.6) (drill 0.3) (layers "F.Cu" "B.Cu") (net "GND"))
 (via (at 106 66) (size 0.6) (drill 0.3) (layers "F.Cu" "B.Cu") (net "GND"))
 (segment (start 107.5 64.5) (end 107.5 64.4) (width 0.2) (layer "B.Cu") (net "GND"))
 (segment (start 116.27 85.5) (end 96.76 85.5) (width 0.2) (layer "B.Cu") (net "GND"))
 (segment (start 96.76 85.5) (end 86.14 74.88) (width 0.2) (layer "B.Cu") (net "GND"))
 (segment (start 106 66) (end 107.5 64.5) (width 0.2) (layer "B.Cu") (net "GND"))
 (segment (start 110.96 87) (end 127.595 87) (width 0.2) (layer "F.Cu") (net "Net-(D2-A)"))
 (segment (start 129.795 89.2) (end 132.335 89.2) (width 0.2) (layer "F.Cu") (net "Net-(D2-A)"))
 (segment (start 127.595 87) (end 129.795 89.2) (width 0.2) (layer "F.Cu") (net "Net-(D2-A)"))
 (segment (start 98.84 74.88) (end 110.96 87) (width 0.2) (layer "F.Cu") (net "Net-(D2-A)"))
 (segment (start 132.335 89.2) (end 133.535 88) (width 0.2) (layer "F.Cu") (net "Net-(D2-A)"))
 (segment (start 103.6 77.1) (end 101.38 74.88) (width 0.2) (layer "F.Cu") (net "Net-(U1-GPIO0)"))
 (segment (start 124.85 76) (end 123.75 77.1) (width 0.2) (layer "F.Cu") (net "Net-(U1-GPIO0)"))
 (segment (start 123.75 77.1) (end 103.6 77.1) (width 0.2) (layer "F.Cu") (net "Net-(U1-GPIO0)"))
 (segment (start 111.42 90) (end 116.27 90) (width 0.2) (layer "F.Cu") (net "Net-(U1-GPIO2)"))
 (segment (start 116.27 90) (end 122.77 90) (width 0.2) (layer "F.Cu") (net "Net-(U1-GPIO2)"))
 (segment (start 96.3 74.88) (end 111.42 90) (width 0.2) (layer "F.Cu") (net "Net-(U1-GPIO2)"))
 (segment (start 83.6 74.88) (end 93.48 65) (width 0.2) (layer "F.Cu") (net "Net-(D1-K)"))
 (segment (start 146.5 64.5) (end 150 68) (width 0.2) (layer "F.Cu") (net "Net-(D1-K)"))
 (segment (start 146.5 53.5) (end 146.5 64.5) (width 0.2) (layer "F.Cu") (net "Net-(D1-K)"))
 (segment (start 93.48 65) (end 124.2925 65) (width 0.2) (layer "F.Cu") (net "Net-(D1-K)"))
 (segment (start 124.2925 65) (end 139 65) (width 0.2) (layer "F.Cu") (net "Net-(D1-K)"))
 (segment (start 141 65) (end 146 65) (width 0.2) (layer "F.Cu") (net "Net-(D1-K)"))
 (segment (start 137.9 48) (end 141 48) (width 0.2) (layer "F.Cu") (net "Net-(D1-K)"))
 (segment (start 141 48) (end 146.5 53.5) (width 0.2) (layer "F.Cu") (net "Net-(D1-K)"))
 (segment (start 146 65) (end 146.5 64.5) (width 0.2) (layer "F.Cu") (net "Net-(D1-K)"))
 (via (at 139 65) (size 0.6) (drill 0.3) (layers "F.Cu" "B.Cu") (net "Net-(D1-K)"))
 (via (at 141 65) (size 0.6) (drill 0.3) (layers "F.Cu" "B.Cu") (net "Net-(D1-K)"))
 (segment (start 139 65) (end 141 65) (width 0.2) (layer "B.Cu") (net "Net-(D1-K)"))
 (segment (start 133.77 74.07) (end 139.84 68) (width 0.2) (layer "F.Cu") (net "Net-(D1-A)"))
 (segment (start 139.84 61.94) (end 137.9 60) (width 0.2) (layer "F.Cu") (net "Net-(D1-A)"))
 (segment (start 139.84 68) (end 139.84 61.94) (width 0.2) (layer "F.Cu") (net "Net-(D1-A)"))
 (segment (start 133.77 76.36) (end 133.77 74.07) (width 0.2) (layer "F.Cu") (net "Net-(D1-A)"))
 (segment (start 130.59 73.5) (end 132.5 75.41) (width 0.2) (layer "F.Cu") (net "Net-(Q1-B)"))
 (segment (start 114.69 76) (end 114.69 73.81) (width 0.2) (layer "F.Cu") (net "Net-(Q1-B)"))
 (segment (start 114.69 73.81) (end 115 73.5) (width 0.2) (layer "F.Cu") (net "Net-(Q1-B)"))
 (segment (start 115 73.5) (end 130.59 73.5) (width 0.2) (layer "F.Cu") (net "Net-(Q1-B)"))
 (segment (start 132.5 75.41) (end 132.5 76.36) (width 0.2) (layer "F.Cu") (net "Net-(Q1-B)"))
 (segment (start 81.8275 54.955) (end 89.5 54.955) (width 0.3) (layer "F.Cu") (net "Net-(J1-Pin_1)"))
 (segment (start 131 44.5) (end 91 44.5) (width 0.3) (layer "F.Cu") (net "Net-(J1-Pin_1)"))
 (segment (start 135.9 54) (end 131 49.1) (width 0.3) (layer "F.Cu") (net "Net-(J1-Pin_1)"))
 (segment (start 89.5 54.955) (end 95.1675 54.955) (width 0.3) (layer "F.Cu") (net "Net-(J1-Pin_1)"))
 (segment (start 91 44.5) (end 89.5 46) (width 0.3) (layer "F.Cu") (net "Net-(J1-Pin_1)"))
 (segment (start 95.1675 54.955) (end 95.2125 55) (width 0.2) (layer "F.Cu") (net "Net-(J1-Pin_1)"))
 (segment (start 89.5 46) (end 89.5 54.955) (width 0.3) (layer "F.Cu") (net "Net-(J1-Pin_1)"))
 (segment (start 131 49.1) (end 131 44.5) (width 0.3) (layer "F.Cu") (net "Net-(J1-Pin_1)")))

